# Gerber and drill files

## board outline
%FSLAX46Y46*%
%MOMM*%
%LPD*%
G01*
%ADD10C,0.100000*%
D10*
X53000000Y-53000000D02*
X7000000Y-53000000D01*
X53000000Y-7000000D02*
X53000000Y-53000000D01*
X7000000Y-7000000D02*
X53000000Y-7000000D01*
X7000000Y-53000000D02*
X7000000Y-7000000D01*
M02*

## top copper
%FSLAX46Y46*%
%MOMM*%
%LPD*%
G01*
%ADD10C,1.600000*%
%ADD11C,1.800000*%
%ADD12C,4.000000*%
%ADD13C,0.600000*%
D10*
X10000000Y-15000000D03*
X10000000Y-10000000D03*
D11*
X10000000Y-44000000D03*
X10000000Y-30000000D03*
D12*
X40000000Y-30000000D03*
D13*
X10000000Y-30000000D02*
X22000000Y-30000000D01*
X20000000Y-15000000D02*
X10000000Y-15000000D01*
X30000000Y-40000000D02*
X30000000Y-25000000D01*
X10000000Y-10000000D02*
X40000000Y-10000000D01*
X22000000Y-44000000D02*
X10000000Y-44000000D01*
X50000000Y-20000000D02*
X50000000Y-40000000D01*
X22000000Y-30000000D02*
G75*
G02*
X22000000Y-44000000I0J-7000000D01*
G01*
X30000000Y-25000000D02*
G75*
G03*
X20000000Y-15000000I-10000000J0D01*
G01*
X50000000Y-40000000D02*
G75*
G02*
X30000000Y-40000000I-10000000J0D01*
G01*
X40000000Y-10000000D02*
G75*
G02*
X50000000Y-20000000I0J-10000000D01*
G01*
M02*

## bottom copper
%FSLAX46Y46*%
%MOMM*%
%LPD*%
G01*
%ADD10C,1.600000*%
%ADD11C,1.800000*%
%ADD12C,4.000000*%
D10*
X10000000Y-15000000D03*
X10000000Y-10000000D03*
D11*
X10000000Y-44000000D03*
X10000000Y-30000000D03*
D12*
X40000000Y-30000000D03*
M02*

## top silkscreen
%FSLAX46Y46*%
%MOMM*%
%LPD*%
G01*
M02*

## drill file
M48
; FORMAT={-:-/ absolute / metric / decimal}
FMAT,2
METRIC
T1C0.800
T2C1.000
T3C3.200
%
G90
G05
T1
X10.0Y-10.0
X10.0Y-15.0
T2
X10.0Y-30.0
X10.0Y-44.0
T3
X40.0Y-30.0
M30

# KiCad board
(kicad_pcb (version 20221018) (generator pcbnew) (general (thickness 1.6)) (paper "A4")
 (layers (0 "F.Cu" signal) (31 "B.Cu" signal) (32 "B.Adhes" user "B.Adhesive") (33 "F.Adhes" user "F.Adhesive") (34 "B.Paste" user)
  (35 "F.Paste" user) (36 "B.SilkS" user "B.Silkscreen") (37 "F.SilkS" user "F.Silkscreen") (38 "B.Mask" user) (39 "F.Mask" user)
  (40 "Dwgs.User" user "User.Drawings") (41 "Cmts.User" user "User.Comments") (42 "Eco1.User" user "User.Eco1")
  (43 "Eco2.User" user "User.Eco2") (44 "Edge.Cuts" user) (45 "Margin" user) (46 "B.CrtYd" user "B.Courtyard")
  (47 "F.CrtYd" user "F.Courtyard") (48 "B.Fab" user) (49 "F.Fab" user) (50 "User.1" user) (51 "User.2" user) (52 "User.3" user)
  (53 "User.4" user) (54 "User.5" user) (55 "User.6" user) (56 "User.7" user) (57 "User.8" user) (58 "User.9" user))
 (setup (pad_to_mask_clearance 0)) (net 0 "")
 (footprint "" (layer "F.Cu") (at 10 15)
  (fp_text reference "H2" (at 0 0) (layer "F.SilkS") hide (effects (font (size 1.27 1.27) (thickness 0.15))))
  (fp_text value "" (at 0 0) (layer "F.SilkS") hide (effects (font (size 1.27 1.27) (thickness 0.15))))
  (pad "" thru_hole circle (at 0 0) (size 1.6 1.6) (drill 0.8) (layers "*.Cu" "*.Mask")))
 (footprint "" (layer "F.Cu") (at 10 10)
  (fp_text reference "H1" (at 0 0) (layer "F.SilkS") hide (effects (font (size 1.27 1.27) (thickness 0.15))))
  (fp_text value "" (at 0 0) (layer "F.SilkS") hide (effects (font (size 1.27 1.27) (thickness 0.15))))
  (pad "" thru_hole circle (at 0 0) (size 1.6 1.6) (drill 0.8) (layers "*.Cu" "*.Mask")))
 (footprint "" (layer "F.Cu") (at 10 44)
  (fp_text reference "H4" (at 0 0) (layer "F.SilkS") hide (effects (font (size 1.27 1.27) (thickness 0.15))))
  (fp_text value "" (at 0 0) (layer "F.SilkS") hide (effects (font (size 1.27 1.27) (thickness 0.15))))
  (pad "" thru_hole circle (at 0 0) (size 1.8 1.8) (drill 1) (layers "*.Cu" "*.Mask")))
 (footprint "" (layer "F.Cu") (at 10 30)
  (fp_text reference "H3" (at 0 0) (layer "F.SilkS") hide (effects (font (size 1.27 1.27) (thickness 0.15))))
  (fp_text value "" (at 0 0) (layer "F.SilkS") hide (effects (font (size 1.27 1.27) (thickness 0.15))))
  (pad "" thru_hole circle (at 0 0) (size 1.8 1.8) (drill 1) (layers "*.Cu" "*.Mask")))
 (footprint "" (layer "F.Cu") (at 40 30)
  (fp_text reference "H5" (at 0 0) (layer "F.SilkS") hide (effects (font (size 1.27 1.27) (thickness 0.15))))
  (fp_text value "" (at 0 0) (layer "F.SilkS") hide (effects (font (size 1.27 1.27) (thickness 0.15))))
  (pad "" thru_hole circle (at 0 0) (size 4 4) (drill 3.2) (layers "*.Cu" "*.Mask")))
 (gr_line (start 53 53) (end 7 53) (stroke (width 0.1) (type default)) (layer "Edge.Cuts"))
 (gr_line (start 53 7) (end 53 53) (stroke (width 0.1) (type default)) (layer "Edge.Cuts"))
 (gr_line (start 7 7) (end 53 7) (stroke (width 0.1) (type default)) (layer "Edge.Cuts"))
 (gr_line (start 7 53) (end 7 7) (stroke (width 0.1) (type default)) (layer "Edge.Cuts"))
 (segment (start 10 30) (end 22 30) (width 0.6) (layer "F.Cu") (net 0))
 (segment (start 20 15) (end 10 15) (width 0.6) (layer "F.Cu") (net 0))
 (segment (start 30 40) (end 30 25) (width 0.6) (layer "F.Cu") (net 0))
 (segment (start 10 10) (end 40 10) (width 0.6) (layer "F.Cu") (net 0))
 (segment (start 22 44) (end 10 44) (width 0.6) (layer "F.Cu") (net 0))
 (segment (start 50 20) (end 50 40) (width 0.6) (layer "F.Cu") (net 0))
 (arc (start 22 30) (mid 29 37) (end 22 44) (width 0.6) (layer "F.Cu") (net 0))
 (arc (start 30 25) (mid 27.071067 17.928932) (end 20 15) (width 0.6) (layer "F.Cu") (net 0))
 (arc (start 50 40) (mid 40 50) (end 30 40) (width 0.6) (layer "F.Cu") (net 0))
 (arc (start 40 10) (mid 47.071067 12.928932) (end 50 20) (width 0.6) (layer "F.Cu") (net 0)))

